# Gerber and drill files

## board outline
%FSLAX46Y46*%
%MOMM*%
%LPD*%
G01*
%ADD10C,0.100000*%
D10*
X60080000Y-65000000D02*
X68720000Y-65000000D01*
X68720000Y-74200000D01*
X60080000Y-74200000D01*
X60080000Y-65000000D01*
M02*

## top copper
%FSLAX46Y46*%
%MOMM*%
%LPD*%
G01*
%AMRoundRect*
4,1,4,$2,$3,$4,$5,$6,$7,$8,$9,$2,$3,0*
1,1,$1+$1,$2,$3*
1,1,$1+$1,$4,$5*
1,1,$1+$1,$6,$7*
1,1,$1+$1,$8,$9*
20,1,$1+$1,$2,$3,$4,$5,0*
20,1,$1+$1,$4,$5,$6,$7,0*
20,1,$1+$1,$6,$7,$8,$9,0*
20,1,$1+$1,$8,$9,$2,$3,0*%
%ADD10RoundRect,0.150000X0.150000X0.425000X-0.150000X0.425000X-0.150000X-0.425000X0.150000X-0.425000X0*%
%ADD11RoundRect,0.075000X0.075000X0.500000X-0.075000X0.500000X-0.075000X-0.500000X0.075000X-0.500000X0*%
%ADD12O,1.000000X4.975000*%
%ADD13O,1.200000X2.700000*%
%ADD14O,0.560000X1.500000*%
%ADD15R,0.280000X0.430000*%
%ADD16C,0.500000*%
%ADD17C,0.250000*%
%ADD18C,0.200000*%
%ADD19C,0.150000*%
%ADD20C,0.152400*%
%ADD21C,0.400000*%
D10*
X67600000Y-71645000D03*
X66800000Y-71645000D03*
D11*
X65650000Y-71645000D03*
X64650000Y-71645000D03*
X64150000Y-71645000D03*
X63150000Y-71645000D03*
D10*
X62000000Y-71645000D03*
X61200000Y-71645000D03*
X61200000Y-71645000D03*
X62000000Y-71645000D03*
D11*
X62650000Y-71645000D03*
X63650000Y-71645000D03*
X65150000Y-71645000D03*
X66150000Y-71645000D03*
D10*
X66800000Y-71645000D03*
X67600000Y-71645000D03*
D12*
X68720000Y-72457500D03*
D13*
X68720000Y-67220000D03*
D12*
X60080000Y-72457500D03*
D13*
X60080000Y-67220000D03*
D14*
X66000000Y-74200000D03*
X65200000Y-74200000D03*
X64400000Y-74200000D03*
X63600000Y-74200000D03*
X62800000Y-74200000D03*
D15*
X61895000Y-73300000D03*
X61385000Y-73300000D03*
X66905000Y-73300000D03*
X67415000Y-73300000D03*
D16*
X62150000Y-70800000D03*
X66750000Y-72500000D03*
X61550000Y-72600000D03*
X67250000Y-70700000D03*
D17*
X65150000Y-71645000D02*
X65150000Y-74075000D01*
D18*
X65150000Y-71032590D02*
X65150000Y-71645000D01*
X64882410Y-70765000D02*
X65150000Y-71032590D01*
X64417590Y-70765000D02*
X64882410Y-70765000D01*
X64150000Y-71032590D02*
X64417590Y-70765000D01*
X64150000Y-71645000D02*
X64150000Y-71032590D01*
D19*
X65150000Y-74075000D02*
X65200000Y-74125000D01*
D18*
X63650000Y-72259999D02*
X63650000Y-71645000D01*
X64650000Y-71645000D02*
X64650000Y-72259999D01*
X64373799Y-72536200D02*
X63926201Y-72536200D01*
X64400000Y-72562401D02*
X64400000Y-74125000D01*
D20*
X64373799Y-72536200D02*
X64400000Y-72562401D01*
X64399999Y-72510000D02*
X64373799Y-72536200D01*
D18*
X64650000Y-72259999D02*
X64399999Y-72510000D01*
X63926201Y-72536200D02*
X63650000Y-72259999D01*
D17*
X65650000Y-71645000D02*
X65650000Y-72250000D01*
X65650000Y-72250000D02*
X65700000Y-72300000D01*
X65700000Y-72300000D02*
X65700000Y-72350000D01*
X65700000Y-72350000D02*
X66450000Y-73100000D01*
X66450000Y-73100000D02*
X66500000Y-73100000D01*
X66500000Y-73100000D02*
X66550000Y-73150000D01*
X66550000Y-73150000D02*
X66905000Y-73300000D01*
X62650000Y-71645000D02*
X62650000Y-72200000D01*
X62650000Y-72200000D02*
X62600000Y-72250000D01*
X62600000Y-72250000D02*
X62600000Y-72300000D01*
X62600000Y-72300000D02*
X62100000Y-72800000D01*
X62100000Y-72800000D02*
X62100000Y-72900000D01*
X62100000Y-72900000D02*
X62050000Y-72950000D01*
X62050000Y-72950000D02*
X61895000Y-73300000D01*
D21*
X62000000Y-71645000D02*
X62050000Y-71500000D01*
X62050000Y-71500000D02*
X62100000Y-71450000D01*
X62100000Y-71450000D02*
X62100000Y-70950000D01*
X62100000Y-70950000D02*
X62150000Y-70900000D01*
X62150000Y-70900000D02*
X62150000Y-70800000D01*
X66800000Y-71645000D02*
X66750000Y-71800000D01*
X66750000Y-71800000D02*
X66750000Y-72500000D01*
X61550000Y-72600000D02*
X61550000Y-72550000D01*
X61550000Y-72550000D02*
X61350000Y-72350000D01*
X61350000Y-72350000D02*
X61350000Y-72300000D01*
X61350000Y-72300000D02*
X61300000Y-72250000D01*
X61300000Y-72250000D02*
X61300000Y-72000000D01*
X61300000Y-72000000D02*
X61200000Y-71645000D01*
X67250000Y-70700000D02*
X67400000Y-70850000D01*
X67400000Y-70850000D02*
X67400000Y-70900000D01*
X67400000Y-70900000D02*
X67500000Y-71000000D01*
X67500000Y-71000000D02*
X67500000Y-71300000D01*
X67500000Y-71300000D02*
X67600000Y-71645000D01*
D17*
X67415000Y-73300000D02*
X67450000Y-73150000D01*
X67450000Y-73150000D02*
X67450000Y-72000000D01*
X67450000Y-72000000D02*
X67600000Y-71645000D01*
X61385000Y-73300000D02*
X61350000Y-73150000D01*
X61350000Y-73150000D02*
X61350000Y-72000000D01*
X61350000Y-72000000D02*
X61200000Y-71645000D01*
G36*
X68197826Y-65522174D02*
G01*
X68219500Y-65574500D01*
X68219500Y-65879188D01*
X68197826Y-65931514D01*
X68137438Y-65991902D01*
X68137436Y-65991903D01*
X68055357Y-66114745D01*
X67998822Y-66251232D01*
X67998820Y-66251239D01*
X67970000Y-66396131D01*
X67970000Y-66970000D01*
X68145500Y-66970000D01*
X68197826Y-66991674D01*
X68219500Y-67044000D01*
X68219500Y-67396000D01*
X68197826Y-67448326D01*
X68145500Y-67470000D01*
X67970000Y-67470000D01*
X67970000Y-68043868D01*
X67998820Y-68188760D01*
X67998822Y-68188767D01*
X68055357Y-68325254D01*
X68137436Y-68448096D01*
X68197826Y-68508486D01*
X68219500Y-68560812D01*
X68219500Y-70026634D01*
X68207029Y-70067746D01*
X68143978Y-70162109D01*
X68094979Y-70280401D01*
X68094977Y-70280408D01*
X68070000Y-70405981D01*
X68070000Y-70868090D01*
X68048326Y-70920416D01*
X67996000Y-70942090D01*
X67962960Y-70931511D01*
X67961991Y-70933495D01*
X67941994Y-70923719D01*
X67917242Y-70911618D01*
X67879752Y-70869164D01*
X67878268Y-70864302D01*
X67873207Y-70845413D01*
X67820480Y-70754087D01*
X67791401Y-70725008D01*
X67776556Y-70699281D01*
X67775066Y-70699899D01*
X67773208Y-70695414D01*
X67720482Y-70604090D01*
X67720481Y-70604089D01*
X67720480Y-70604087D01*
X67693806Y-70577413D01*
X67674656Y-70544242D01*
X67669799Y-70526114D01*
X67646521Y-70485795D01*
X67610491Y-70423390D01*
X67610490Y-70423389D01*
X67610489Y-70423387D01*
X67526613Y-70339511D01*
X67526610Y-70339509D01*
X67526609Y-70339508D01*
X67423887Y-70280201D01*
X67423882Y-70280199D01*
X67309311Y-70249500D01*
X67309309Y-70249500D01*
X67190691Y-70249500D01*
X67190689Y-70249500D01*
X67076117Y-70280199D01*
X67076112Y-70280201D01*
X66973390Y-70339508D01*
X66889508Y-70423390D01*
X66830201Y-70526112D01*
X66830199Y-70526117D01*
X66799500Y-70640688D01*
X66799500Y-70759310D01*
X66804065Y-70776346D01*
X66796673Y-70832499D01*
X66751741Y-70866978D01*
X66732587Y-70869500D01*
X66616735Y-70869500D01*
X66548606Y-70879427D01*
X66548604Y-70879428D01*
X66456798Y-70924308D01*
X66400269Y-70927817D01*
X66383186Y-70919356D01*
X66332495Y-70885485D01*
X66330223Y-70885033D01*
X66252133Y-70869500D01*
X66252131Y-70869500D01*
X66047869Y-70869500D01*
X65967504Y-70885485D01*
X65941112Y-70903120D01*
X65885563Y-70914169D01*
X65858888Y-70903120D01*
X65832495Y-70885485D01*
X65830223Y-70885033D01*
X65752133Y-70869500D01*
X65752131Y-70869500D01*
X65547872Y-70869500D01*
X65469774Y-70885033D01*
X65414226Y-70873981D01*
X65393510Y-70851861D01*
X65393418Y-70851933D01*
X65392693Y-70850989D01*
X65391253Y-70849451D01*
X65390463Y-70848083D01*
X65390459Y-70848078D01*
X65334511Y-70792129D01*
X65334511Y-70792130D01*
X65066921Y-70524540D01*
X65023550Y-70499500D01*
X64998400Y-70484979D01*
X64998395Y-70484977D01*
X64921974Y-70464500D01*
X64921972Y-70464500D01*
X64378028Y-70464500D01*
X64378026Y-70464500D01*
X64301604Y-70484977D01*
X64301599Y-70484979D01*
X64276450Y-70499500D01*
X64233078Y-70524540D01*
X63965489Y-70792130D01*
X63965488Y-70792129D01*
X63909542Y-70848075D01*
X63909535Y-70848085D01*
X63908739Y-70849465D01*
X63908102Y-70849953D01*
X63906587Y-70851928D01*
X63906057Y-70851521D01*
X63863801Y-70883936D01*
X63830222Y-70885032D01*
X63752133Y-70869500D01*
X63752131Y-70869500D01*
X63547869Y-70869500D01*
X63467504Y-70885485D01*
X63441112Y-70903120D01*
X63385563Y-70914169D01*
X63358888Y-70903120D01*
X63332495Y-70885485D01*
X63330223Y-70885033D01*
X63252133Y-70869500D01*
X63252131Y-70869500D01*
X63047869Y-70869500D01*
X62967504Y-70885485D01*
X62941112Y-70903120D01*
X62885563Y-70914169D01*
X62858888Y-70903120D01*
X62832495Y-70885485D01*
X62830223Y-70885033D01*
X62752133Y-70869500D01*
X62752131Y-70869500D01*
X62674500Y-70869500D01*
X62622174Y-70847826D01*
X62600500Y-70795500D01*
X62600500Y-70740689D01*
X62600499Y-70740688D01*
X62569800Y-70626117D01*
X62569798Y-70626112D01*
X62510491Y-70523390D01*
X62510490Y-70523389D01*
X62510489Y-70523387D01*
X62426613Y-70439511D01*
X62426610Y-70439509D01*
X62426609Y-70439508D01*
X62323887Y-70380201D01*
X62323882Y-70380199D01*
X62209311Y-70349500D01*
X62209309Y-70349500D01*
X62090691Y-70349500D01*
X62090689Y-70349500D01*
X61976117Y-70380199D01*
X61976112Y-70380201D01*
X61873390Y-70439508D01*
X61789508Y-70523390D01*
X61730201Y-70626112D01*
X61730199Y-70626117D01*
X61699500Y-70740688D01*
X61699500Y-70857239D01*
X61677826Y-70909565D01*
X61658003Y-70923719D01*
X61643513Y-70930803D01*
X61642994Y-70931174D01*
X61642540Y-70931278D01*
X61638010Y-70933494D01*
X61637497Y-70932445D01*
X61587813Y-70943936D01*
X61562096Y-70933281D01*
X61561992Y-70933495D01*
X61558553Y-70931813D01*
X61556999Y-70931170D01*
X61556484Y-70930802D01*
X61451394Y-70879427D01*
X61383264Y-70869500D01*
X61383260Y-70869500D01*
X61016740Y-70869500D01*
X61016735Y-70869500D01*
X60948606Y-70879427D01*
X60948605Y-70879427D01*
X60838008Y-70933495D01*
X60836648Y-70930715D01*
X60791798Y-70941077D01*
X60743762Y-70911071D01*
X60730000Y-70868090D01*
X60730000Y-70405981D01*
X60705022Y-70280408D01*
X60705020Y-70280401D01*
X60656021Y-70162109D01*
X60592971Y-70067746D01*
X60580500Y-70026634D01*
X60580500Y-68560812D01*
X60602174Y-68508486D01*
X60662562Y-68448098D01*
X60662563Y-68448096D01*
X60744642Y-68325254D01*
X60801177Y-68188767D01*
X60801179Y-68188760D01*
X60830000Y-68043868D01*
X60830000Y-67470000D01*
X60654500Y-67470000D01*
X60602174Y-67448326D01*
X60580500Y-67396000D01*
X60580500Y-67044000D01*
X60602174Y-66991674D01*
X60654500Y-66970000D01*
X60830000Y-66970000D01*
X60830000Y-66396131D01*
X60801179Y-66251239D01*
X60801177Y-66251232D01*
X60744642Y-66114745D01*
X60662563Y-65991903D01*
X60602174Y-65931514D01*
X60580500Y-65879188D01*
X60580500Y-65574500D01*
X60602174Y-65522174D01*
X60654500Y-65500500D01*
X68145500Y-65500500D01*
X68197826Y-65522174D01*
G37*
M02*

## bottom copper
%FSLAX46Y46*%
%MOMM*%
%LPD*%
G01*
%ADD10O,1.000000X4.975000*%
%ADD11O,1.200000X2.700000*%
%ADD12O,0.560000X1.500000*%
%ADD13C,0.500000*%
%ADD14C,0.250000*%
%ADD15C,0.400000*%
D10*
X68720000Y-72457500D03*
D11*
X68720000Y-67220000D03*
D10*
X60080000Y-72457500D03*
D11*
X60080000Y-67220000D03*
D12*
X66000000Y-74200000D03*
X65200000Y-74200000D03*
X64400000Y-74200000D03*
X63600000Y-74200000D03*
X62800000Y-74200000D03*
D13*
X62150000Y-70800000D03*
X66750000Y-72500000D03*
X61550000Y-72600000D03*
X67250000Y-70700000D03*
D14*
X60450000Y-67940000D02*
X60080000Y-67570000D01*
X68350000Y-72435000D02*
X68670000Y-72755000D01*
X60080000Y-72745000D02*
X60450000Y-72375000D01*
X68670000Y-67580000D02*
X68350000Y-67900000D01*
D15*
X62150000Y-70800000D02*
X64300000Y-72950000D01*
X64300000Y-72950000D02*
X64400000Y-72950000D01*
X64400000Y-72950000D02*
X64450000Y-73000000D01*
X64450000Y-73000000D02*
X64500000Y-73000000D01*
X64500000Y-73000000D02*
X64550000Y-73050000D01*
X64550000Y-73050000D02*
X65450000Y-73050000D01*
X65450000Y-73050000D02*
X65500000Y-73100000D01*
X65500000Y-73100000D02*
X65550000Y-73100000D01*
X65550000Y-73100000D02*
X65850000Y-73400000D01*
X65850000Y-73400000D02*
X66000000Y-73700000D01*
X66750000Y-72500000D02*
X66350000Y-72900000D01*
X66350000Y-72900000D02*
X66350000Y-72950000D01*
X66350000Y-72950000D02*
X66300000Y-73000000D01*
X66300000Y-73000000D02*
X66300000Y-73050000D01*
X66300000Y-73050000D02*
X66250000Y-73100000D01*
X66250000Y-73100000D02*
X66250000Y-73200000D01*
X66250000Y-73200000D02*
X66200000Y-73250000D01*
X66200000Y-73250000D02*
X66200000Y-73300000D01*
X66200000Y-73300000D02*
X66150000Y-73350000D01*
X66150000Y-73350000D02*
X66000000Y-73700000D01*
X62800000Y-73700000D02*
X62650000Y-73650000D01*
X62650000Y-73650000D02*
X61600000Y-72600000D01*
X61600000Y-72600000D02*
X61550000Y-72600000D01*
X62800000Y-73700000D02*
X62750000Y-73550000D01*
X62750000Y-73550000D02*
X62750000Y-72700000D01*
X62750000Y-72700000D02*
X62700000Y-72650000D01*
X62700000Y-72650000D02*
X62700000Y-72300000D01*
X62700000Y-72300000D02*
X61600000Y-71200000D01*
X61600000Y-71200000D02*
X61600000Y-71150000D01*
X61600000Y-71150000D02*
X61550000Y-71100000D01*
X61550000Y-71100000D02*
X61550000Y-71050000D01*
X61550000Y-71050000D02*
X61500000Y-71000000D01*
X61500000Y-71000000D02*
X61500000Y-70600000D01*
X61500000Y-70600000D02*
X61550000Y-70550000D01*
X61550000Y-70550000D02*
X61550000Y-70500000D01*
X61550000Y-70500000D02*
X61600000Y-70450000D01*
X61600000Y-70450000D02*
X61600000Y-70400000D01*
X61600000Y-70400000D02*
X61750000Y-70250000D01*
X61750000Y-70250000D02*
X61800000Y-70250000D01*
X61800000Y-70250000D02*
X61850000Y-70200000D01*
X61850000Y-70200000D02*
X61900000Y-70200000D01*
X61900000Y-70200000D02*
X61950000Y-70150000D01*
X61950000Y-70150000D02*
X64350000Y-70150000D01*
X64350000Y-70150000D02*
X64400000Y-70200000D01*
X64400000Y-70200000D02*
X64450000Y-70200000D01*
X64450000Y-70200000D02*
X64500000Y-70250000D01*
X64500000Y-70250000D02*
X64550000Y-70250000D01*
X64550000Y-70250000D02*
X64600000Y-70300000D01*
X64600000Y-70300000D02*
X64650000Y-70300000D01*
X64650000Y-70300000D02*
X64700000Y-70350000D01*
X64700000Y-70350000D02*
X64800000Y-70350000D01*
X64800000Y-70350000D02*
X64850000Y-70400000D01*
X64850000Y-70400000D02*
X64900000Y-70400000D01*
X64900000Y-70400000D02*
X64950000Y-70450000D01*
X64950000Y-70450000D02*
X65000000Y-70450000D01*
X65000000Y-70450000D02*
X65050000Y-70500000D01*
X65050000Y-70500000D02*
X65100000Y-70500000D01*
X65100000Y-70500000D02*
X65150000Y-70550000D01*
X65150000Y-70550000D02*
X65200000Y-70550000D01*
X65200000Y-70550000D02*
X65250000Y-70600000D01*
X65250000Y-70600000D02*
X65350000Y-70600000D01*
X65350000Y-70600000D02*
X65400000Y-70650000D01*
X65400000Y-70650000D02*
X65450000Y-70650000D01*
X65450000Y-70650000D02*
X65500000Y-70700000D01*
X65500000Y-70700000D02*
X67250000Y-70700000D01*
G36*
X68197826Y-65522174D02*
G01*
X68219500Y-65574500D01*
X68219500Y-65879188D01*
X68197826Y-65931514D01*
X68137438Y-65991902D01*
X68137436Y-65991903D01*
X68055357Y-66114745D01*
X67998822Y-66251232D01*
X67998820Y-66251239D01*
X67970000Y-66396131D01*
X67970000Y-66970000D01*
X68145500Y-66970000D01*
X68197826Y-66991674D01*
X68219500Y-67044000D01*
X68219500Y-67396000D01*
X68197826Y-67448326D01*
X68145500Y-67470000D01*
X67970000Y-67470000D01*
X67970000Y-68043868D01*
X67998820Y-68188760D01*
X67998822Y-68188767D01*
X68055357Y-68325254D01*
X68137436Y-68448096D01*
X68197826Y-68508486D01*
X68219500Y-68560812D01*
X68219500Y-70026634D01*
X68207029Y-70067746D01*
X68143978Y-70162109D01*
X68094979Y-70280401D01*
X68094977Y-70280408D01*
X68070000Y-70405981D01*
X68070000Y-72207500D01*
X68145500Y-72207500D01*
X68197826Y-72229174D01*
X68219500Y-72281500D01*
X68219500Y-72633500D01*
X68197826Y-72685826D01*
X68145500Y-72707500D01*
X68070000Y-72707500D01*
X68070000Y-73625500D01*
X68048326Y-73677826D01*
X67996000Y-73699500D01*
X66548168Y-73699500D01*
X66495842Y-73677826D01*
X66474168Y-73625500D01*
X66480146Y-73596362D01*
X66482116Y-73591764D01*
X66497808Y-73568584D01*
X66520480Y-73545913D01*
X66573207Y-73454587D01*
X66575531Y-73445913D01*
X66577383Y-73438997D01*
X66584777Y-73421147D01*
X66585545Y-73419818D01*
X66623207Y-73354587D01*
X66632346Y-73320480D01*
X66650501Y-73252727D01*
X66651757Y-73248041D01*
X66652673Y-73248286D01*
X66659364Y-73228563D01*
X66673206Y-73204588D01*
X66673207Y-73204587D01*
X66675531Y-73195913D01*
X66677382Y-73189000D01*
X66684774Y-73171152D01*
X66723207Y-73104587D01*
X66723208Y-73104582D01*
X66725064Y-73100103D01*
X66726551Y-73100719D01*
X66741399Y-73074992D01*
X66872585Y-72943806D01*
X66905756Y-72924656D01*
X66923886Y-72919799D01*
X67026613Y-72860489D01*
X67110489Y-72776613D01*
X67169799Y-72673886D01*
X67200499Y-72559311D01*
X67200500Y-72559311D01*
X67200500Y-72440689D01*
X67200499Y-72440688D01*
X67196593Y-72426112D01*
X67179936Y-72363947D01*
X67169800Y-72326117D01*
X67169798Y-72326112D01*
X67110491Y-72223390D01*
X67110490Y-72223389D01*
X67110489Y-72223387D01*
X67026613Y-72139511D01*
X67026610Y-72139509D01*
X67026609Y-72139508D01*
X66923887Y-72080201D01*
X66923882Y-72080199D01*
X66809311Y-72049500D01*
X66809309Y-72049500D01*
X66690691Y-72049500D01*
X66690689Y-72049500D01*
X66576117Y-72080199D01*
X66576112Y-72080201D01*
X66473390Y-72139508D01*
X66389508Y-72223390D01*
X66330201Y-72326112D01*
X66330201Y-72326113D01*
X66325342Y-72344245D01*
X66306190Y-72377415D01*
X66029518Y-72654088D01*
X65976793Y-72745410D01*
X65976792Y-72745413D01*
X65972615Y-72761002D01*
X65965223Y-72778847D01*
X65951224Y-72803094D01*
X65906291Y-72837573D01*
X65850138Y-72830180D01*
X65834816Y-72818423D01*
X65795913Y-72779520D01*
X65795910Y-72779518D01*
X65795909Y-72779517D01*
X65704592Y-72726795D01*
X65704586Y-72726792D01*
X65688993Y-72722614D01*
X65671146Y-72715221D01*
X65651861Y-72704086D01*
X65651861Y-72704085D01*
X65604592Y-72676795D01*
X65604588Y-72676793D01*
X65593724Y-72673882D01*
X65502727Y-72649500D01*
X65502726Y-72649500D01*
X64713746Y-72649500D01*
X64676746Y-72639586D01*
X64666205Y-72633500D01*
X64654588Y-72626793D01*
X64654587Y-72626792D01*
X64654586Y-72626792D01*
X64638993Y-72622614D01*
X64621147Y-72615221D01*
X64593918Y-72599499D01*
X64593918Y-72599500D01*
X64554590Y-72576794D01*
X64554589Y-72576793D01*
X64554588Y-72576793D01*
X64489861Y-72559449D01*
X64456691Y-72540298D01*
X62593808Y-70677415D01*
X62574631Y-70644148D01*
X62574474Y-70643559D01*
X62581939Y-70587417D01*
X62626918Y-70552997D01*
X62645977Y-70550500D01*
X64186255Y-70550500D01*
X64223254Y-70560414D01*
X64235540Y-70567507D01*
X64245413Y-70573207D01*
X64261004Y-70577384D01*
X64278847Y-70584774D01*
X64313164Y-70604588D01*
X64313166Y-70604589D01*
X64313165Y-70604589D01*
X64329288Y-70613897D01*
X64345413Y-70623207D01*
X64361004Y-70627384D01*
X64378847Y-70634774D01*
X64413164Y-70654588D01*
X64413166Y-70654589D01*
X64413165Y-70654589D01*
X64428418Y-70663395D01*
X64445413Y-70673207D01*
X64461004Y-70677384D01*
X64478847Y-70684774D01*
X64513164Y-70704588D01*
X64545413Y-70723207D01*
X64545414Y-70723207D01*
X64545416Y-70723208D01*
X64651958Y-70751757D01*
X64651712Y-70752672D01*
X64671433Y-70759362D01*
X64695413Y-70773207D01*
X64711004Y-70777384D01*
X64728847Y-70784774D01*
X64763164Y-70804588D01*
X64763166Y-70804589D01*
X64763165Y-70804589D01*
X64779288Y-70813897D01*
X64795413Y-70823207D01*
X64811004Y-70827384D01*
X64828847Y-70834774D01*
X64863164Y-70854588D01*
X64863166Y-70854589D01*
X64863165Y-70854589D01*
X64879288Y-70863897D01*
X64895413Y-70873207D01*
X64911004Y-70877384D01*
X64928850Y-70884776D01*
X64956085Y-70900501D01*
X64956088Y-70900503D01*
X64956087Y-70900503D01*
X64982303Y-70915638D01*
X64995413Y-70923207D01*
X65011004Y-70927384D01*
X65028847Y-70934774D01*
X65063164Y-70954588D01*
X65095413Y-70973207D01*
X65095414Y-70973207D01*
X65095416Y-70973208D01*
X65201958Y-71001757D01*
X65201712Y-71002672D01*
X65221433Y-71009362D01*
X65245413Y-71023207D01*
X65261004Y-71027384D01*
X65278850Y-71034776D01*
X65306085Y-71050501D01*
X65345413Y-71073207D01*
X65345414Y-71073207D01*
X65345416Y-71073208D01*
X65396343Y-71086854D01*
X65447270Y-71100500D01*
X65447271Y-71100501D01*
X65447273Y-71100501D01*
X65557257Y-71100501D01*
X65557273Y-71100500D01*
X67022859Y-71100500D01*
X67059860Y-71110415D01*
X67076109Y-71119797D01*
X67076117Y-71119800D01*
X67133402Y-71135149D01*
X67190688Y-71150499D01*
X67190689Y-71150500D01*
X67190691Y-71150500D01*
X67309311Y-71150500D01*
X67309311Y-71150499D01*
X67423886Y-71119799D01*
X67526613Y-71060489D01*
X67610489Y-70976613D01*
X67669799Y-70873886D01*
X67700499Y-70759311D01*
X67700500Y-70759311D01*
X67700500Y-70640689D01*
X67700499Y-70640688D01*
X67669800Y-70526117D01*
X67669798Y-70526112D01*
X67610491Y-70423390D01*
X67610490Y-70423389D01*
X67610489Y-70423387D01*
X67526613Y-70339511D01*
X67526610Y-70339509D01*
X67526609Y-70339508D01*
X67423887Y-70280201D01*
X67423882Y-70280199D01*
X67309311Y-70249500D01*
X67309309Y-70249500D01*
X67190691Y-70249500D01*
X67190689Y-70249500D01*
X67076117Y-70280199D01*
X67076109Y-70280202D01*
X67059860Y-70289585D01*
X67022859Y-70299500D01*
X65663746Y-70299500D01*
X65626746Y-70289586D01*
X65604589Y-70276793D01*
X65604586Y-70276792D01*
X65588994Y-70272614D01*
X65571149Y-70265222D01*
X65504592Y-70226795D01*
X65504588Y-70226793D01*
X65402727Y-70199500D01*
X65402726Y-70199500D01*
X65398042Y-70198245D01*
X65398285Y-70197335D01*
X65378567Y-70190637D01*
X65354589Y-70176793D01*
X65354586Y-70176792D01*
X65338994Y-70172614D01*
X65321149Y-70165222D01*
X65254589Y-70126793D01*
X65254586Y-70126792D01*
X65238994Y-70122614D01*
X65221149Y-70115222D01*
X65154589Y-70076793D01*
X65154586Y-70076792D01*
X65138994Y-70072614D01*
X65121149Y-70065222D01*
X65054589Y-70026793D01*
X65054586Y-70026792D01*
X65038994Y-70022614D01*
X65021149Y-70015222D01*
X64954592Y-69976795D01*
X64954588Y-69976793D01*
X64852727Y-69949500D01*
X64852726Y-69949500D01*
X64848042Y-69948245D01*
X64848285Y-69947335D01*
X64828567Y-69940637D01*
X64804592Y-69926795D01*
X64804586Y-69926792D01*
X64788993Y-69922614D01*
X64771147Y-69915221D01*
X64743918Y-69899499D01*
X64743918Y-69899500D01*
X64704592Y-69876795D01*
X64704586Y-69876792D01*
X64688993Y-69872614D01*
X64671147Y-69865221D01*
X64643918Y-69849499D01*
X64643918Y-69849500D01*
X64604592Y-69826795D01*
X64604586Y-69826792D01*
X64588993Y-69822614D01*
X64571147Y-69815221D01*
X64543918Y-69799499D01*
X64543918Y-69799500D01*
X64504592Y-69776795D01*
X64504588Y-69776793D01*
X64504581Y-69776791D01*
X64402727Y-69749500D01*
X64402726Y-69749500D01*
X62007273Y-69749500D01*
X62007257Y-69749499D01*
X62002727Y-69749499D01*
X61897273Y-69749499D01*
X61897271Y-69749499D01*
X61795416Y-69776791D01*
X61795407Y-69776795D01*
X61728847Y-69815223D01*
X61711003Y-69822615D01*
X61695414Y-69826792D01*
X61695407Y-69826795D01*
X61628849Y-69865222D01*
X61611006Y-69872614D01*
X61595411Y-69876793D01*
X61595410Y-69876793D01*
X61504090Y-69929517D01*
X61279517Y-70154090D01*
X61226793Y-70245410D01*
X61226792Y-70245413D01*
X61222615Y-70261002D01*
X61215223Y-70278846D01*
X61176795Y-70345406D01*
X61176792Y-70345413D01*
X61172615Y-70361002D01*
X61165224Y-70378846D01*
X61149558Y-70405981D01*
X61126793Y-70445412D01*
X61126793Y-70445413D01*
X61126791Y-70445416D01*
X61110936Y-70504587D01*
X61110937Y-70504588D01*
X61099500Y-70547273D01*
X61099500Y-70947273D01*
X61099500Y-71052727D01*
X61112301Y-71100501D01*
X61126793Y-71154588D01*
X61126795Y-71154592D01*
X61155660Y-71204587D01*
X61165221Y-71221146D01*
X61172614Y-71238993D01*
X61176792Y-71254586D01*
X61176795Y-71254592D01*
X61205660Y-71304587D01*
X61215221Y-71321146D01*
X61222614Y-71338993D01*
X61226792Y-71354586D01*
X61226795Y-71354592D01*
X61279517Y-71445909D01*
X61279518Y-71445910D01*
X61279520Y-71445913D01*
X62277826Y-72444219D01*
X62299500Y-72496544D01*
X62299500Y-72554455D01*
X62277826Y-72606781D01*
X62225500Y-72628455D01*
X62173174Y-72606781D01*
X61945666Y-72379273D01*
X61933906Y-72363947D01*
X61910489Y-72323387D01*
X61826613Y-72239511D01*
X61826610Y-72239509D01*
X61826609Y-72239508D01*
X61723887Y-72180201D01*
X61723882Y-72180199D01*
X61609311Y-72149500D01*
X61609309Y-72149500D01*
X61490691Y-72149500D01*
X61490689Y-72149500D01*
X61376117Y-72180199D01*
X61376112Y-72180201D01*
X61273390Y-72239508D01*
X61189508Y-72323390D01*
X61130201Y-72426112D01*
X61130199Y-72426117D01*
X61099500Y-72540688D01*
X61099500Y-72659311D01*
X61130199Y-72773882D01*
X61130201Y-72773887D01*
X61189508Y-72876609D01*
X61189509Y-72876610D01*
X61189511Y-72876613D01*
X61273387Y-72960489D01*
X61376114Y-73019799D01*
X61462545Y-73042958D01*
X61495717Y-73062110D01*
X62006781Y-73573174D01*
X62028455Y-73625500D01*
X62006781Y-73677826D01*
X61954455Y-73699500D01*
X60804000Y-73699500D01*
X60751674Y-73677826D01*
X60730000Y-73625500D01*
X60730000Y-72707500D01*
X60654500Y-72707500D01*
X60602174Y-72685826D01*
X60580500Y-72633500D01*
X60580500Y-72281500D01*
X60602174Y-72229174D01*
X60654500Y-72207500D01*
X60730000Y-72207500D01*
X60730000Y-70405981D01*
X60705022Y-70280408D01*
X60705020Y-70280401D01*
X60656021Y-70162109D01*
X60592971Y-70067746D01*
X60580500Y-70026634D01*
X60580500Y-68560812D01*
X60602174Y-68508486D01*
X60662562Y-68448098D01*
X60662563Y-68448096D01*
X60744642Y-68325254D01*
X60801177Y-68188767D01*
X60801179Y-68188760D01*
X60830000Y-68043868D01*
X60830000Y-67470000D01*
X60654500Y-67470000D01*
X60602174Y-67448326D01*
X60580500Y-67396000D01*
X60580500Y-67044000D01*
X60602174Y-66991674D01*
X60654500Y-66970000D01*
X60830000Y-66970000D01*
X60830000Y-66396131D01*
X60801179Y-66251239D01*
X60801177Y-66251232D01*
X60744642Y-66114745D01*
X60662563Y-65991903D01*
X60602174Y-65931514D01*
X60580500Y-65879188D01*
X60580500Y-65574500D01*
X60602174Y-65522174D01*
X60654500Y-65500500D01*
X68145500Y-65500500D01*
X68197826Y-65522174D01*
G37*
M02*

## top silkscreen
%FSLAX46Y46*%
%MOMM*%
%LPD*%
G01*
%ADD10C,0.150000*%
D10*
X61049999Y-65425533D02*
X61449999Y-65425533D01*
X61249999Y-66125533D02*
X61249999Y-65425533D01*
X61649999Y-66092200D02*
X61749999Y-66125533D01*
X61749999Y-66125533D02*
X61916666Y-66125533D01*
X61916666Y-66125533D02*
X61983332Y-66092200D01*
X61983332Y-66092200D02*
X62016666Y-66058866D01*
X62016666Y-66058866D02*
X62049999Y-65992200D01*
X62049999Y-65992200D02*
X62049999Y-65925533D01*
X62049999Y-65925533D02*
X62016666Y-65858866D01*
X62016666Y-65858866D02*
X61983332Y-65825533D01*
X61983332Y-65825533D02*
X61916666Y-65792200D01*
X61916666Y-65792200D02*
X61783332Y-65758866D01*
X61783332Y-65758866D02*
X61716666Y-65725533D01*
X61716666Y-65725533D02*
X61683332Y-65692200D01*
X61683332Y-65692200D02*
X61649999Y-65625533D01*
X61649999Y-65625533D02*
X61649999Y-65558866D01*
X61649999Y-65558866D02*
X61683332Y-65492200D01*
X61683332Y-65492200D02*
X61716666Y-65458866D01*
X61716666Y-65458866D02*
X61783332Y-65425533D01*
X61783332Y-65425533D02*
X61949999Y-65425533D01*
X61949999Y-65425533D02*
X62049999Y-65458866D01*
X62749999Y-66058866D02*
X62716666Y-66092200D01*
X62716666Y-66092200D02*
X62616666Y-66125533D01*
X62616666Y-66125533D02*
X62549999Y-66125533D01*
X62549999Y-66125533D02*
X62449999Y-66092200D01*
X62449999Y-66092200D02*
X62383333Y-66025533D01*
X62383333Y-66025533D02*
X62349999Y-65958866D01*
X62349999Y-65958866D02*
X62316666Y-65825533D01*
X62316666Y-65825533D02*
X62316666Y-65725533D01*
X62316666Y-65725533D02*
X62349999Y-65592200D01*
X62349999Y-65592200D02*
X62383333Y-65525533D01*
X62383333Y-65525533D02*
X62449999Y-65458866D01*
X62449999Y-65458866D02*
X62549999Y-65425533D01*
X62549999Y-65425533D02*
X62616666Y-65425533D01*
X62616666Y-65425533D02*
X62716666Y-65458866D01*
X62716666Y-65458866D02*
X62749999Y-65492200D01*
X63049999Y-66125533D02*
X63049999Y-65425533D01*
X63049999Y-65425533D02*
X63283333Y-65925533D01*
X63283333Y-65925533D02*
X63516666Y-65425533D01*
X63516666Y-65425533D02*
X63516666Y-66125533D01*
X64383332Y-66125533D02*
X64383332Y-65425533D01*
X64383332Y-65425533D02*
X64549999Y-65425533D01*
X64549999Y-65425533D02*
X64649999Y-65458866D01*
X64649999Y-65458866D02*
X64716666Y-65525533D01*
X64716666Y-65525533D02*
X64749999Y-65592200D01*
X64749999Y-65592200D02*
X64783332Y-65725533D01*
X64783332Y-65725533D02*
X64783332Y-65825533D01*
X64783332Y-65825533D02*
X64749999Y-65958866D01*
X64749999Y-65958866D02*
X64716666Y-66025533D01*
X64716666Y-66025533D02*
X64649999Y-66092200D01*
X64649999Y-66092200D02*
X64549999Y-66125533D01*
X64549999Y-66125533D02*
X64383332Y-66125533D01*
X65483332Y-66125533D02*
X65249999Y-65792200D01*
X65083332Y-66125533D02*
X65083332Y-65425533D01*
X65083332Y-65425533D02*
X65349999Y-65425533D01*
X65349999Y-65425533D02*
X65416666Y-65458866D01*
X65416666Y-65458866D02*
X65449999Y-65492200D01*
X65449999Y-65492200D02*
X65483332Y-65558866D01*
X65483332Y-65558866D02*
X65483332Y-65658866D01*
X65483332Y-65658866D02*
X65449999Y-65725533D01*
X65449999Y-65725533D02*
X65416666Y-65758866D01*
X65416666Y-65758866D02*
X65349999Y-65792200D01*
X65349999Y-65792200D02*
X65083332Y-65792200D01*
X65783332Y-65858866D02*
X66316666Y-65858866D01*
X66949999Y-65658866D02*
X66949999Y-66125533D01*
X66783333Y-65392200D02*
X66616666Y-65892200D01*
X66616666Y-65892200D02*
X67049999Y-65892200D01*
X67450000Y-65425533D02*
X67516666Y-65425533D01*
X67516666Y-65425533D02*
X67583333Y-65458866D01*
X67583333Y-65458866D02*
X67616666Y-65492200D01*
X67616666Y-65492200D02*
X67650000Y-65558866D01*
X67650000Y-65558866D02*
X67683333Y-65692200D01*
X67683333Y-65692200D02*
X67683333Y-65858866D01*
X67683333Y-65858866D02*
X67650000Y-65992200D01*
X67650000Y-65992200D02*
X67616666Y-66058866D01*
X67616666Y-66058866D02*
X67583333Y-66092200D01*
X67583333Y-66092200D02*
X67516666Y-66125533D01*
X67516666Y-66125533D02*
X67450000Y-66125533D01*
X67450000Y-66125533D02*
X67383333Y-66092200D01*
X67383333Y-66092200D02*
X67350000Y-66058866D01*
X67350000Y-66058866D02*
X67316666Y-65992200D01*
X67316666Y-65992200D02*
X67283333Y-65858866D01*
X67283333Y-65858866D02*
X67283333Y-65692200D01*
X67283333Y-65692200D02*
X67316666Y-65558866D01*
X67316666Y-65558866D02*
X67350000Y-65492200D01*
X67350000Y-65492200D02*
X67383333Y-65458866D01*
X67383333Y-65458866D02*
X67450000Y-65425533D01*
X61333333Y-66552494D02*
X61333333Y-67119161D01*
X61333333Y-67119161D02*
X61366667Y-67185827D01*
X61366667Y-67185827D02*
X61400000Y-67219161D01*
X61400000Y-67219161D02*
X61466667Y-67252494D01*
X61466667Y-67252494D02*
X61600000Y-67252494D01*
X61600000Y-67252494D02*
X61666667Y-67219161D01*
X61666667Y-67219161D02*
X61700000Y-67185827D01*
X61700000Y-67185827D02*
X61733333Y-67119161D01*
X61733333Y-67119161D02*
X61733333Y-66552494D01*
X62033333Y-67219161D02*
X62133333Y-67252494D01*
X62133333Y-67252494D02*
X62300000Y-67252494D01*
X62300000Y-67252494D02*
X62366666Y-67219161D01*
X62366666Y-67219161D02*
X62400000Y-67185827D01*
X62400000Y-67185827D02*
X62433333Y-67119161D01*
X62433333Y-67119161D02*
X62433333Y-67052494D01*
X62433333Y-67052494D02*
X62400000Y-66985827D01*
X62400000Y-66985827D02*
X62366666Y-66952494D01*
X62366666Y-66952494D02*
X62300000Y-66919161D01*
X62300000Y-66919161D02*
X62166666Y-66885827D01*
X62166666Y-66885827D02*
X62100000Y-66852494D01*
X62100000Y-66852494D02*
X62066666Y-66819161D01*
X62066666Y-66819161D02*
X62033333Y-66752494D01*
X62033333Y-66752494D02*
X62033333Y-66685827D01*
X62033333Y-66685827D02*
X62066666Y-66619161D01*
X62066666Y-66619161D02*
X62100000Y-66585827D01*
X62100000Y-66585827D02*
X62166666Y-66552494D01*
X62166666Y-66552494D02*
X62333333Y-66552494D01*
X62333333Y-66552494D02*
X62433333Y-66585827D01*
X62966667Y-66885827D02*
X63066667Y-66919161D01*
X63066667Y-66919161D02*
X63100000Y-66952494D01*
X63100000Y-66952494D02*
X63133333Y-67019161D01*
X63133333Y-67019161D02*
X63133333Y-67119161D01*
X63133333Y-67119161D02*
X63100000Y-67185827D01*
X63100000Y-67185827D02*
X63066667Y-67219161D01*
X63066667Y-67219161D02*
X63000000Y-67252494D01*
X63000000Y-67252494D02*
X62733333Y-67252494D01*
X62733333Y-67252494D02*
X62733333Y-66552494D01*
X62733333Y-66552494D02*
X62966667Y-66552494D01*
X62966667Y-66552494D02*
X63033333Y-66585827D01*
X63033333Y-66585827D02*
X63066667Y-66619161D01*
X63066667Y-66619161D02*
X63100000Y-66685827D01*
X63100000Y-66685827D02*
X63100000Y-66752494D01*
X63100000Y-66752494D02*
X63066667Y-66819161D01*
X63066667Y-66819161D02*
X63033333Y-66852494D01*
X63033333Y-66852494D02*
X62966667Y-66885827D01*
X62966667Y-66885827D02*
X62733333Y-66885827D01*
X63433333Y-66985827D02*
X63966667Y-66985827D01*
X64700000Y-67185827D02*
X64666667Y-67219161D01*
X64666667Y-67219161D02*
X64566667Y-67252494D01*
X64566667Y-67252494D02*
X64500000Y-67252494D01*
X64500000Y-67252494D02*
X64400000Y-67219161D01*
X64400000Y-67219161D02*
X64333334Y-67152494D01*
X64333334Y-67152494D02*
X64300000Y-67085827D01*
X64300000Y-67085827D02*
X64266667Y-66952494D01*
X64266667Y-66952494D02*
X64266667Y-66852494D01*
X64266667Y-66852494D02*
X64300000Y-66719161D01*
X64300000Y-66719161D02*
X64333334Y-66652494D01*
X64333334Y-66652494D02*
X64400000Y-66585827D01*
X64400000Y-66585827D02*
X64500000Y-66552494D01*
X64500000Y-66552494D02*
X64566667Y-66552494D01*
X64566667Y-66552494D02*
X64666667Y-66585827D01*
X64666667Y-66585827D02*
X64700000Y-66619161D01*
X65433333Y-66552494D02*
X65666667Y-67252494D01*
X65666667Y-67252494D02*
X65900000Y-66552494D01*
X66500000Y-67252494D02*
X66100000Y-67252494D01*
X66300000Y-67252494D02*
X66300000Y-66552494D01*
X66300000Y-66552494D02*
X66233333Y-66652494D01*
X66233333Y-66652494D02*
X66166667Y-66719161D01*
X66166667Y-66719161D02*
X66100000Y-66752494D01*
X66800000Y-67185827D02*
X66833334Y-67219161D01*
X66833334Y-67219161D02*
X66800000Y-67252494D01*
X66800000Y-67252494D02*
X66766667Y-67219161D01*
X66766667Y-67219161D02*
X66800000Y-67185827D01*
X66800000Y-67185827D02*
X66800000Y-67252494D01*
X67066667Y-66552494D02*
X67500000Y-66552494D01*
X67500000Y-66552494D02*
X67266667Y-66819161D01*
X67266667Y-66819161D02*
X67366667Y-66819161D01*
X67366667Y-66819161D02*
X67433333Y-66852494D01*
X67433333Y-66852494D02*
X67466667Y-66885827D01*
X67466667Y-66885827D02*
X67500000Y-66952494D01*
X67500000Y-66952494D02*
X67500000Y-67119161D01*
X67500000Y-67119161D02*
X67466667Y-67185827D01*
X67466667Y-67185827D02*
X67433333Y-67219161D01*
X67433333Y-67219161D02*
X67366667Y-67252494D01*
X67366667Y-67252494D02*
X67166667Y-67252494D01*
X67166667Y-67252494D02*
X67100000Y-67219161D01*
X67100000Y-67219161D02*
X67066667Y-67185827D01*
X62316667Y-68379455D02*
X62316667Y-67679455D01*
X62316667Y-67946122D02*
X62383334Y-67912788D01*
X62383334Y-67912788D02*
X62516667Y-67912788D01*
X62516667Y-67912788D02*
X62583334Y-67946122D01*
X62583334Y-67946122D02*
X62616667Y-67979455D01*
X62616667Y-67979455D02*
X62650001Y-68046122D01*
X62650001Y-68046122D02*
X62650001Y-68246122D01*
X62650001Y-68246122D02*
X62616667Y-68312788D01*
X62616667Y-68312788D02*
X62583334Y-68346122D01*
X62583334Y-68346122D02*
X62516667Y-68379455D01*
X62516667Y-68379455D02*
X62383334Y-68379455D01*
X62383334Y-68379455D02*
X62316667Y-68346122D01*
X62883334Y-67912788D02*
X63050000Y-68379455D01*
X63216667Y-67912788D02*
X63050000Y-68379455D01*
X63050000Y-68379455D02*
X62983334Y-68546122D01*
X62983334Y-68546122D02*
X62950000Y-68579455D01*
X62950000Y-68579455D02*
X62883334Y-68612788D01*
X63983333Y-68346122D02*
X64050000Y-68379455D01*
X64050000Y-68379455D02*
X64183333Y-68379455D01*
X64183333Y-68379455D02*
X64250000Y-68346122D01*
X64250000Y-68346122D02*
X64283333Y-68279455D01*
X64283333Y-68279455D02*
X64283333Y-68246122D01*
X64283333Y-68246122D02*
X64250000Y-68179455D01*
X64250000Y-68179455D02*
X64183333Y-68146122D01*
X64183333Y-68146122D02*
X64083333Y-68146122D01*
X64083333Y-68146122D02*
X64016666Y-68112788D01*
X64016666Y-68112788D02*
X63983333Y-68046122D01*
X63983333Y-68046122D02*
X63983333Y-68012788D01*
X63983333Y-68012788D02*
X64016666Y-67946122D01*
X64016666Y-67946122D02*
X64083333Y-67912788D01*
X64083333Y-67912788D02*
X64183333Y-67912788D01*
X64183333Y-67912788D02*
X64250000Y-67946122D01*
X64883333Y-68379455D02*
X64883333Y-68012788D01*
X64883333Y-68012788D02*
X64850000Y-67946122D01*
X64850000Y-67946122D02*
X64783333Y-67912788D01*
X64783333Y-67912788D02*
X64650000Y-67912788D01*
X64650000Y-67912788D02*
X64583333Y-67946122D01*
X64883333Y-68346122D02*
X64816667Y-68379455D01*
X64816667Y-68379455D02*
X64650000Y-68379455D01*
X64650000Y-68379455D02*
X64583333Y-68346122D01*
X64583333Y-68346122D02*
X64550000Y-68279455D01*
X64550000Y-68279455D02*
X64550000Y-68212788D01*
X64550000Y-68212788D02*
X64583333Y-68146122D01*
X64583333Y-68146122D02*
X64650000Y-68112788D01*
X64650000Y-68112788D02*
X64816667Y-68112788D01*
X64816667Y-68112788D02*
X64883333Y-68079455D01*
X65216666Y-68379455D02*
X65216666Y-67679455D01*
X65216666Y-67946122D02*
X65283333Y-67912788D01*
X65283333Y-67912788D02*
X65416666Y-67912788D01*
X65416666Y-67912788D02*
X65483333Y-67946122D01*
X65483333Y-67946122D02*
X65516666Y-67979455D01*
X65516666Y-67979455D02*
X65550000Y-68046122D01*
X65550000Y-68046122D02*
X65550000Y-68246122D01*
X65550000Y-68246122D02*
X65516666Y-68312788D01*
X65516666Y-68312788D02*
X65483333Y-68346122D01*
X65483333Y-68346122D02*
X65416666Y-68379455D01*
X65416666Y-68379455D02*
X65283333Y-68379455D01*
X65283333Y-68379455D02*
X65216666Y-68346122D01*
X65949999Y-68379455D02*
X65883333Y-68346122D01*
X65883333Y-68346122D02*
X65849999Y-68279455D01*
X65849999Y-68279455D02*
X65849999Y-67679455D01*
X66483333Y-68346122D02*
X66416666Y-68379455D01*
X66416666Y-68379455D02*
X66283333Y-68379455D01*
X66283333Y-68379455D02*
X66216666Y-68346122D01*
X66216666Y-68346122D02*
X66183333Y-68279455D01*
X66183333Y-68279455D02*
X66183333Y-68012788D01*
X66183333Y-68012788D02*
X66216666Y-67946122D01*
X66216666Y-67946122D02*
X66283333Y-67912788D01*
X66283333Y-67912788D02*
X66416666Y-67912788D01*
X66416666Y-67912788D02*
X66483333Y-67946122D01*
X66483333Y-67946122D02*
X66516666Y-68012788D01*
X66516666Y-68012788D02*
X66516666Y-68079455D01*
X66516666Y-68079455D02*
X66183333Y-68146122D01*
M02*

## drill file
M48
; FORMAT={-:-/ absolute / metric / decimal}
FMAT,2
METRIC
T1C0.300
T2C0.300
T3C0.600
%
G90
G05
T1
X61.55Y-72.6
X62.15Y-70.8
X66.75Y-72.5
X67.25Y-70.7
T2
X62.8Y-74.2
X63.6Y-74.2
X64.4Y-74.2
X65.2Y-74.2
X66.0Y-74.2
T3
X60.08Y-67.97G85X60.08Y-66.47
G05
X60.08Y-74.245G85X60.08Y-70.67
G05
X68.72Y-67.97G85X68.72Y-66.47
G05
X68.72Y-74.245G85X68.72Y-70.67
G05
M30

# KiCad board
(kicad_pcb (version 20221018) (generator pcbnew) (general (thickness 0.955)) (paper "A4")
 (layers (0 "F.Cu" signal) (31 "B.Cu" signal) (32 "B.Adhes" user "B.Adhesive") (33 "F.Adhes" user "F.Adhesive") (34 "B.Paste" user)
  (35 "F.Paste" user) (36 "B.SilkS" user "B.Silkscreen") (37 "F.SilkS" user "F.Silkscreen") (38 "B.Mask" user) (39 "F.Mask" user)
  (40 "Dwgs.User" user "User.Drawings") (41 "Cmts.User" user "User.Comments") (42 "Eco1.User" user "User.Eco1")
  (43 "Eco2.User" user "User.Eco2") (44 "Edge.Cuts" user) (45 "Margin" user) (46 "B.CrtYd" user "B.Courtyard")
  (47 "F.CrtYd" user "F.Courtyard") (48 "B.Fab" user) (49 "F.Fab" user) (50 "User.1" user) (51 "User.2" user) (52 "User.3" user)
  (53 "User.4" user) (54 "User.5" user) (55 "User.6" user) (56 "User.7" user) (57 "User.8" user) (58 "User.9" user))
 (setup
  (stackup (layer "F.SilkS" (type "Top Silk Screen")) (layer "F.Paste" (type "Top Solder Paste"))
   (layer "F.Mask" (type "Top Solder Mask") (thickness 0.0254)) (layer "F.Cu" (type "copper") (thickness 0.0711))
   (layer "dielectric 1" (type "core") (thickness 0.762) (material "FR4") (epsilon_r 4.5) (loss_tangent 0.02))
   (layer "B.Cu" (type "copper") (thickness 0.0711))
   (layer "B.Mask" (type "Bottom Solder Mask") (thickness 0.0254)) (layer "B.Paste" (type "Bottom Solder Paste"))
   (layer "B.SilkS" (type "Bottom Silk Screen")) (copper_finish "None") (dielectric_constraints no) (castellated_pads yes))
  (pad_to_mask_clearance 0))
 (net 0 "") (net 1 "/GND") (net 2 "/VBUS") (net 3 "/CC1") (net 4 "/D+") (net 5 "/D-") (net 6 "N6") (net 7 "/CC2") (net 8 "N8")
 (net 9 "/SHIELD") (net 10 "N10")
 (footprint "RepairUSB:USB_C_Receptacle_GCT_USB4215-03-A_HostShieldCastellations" (layer "F.Cu") (at 64.4 68.645 180)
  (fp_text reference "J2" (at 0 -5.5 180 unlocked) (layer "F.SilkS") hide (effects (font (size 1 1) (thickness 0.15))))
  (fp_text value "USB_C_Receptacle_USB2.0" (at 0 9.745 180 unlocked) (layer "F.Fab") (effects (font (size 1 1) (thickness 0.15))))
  (pad "A1" smd roundrect (at -3.2 -3 180) (size 0.6 1.15) (layers "F.Cu" "F.Paste" "F.Mask") (roundrect_rratio 0.25) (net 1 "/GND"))
  (pad "A4" smd roundrect (at -2.4 -3 180) (size 0.6 1.15) (layers "F.Cu" "F.Paste" "F.Mask") (roundrect_rratio 0.25) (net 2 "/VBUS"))
  (pad "A5" smd roundrect (at -1.25 -3 180) (size 0.3 1.15) (layers "F.Cu" "F.Paste" "F.Mask") (roundrect_rratio 0.25) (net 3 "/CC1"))
  (pad "A6" smd roundrect (at -0.25 -3 180) (size 0.3 1.15) (layers "F.Cu" "F.Paste" "F.Mask") (roundrect_rratio 0.25) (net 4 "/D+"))
  (pad "A7" smd roundrect (at 0.25 -3 180) (size 0.3 1.15) (layers "F.Cu" "F.Paste" "F.Mask") (roundrect_rratio 0.25) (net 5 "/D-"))
  (pad "A8" smd roundrect (at 1.25 -3 180) (size 0.3 1.15) (layers "F.Cu" "F.Paste" "F.Mask") (roundrect_rratio 0.25) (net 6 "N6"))
  (pad "A9" smd roundrect (at 2.4 -3 180) (size 0.6 1.15) (layers "F.Cu" "F.Paste" "F.Mask") (roundrect_rratio 0.25) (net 2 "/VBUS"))
  (pad "A12" smd roundrect (at 3.2 -3 180) (size 0.6 1.15) (layers "F.Cu" "F.Paste" "F.Mask") (roundrect_rratio 0.25) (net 1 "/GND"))
  (pad "B1" smd roundrect (at 3.2 -3 180) (size 0.6 1.15) (layers "F.Cu" "F.Paste" "F.Mask") (roundrect_rratio 0.25) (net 1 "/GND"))
  (pad "B4" smd roundrect (at 2.4 -3 180) (size 0.6 1.15) (layers "F.Cu" "F.Paste" "F.Mask") (roundrect_rratio 0.25) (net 2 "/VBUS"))
  (pad "B5" smd roundrect (at 1.75 -3 180) (size 0.3 1.15) (layers "F.Cu" "F.Paste" "F.Mask") (roundrect_rratio 0.25) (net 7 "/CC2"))
  (pad "B6" smd roundrect (at 0.75 -3 180) (size 0.3 1.15) (layers "F.Cu" "F.Paste" "F.Mask") (roundrect_rratio 0.25) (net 4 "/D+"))
  (pad "B7" smd roundrect (at -0.75 -3 180) (size 0.3 1.15) (layers "F.Cu" "F.Paste" "F.Mask") (roundrect_rratio 0.25) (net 5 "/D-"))
  (pad "B8" smd roundrect (at -1.75 -3 180) (size 0.3 1.15) (layers "F.Cu" "F.Paste" "F.Mask") (roundrect_rratio 0.25) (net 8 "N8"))
  (pad "B9" smd roundrect (at -2.4 -3 180) (size 0.6 1.15) (layers "F.Cu" "F.Paste" "F.Mask") (roundrect_rratio 0.25) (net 2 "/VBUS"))
  (pad "B12" smd roundrect (at -3.2 -3 180) (size 0.6 1.15) (layers "F.Cu" "F.Paste" "F.Mask") (roundrect_rratio 0.25) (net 1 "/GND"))
  (pad "S1" thru_hole oval (at -4.32 -3.8125 180) (size 1 4.975) (drill oval 0.6 4.175) (layers "*.Cu" "*.Mask" "F.Paste") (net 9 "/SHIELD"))
  (pad "S1" thru_hole oval (at -4.32 1.425 180) (size 1.2 2.7) (drill oval 0.6 2.1) (layers "*.Cu" "*.Mask" "F.Paste") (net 9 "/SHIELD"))
  (pad "S1" thru_hole oval (at 4.32 -3.8125 180) (size 1 4.975) (drill oval 0.6 4.175) (layers "*.Cu" "*.Mask" "F.Paste") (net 9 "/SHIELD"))
  (pad "S1" thru_hole oval (at 4.32 1.425 180) (size 1.2 2.7) (drill oval 0.6 2.1) (layers "*.Cu" "*.Mask" "F.Paste") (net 9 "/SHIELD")))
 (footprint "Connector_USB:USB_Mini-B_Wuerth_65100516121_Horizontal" (layer "F.Cu") (at 64.4 72.35 180)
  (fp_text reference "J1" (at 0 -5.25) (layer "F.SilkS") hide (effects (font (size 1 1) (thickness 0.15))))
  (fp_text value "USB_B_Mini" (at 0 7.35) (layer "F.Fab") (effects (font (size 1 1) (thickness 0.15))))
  (pad "1" thru_hole oval (at -1.6 -1.85 180) (size 0.56 1.5) (drill 0.3) (layers "*.Cu" "*.Mask") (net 2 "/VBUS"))
  (pad "2" thru_hole oval (at -0.8 -1.85 180) (size 0.56 1.5) (drill 0.3) (layers "*.Cu" "*.Mask") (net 5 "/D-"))
  (pad "3" thru_hole oval (at 0 -1.85 180) (size 0.56 1.5) (drill 0.3) (layers "*.Cu" "*.Mask") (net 4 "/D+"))
  (pad "4" thru_hole oval (at 0.8 -1.85 180) (size 0.56 1.5) (drill 0.3) (layers "*.Cu" "*.Mask") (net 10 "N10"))
  (pad "5" thru_hole oval (at 1.6 -1.85 180) (size 0.56 1.5) (drill 0.3) (layers "*.Cu" "*.Mask") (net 1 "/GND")))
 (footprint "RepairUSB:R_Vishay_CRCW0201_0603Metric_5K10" (layer "F.Cu") (at 61.64 73.3 180)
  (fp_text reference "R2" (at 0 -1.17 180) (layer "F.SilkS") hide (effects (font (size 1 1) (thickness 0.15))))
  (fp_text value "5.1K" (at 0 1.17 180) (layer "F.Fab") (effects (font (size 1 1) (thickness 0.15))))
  (pad "1" smd rect (at -0.255 0 180) (size 0.28 0.43) (layers "F.Cu" "F.Paste" "F.Mask") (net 7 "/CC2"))
  (pad "2" smd rect (at 0.255 0 180) (size 0.28 0.43) (layers "F.Cu" "F.Paste" "F.Mask") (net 1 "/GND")))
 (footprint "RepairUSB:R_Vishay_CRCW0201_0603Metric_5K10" (layer "F.Cu") (at 67.16 73.3)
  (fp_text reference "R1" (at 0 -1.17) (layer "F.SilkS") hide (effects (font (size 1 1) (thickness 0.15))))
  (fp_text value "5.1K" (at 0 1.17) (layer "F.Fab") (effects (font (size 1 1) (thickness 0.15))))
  (pad "1" smd rect (at -0.255 0) (size 0.28 0.43) (layers "F.Cu" "F.Paste" "F.Mask") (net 3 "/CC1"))
  (pad "2" smd rect (at 0.255 0) (size 0.28 0.43) (layers "F.Cu" "F.Paste" "F.Mask") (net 1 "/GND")))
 (gr_rect locked (start 60.08 65) (end 68.72 74.2) (stroke (width 0.1) (type default)) (fill none) (layer "Edge.Cuts"))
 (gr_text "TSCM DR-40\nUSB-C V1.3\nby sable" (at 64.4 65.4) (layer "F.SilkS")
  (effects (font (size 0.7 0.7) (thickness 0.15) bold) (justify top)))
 (segment (start 65.15 71.645) (end 65.15 74.075) (width 0.25) (layer "F.Cu") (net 5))
 (segment (start 65.15 71.03259) (end 65.15 71.645) (width 0.2) (layer "F.Cu") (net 5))
 (segment (start 64.88241 70.765) (end 65.15 71.03259) (width 0.2) (layer "F.Cu") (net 5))
 (segment (start 64.41759 70.765) (end 64.88241 70.765) (width 0.2) (layer "F.Cu") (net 5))
 (segment (start 64.15 71.03259) (end 64.41759 70.765) (width 0.2) (layer "F.Cu") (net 5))
 (segment (start 64.15 71.645) (end 64.15 71.03259) (width 0.2) (layer "F.Cu") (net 5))
 (segment (start 65.15 74.075) (end 65.2 74.125) (width 0.15) (layer "F.Cu") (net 5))
 (segment (start 63.65 72.259999) (end 63.65 71.645) (width 0.2) (layer "F.Cu") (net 4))
 (segment (start 64.65 71.645) (end 64.65 72.259999) (width 0.2) (layer "F.Cu") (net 4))
 (segment (start 64.373799 72.5362) (end 63.926201 72.5362) (width 0.2) (layer "F.Cu") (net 4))
 (segment (start 64.4 72.562401) (end 64.4 74.125) (width 0.2) (layer "F.Cu") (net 4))
 (segment (start 64.373799 72.5362) (end 64.4 72.562401) (width 0.1524) (layer "F.Cu") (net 4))
 (segment (start 64.399999 72.51) (end 64.373799 72.5362) (width 0.1524) (layer "F.Cu") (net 4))
 (segment (start 64.65 72.259999) (end 64.399999 72.51) (width 0.2) (layer "F.Cu") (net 4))
 (segment (start 63.926201 72.5362) (end 63.65 72.259999) (width 0.2) (layer "F.Cu") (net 4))
 (segment (start 60.45 67.94) (end 60.08 67.57) (width 0.25) (layer "B.Cu") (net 9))
 (segment (start 68.35 72.435) (end 68.67 72.755) (width 0.25) (layer "B.Cu") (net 9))
 (segment (start 60.08 72.745) (end 60.45 72.375) (width 0.25) (layer "B.Cu") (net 9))
 (segment (start 68.67 67.58) (end 68.35 67.9) (width 0.25) (layer "B.Cu") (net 9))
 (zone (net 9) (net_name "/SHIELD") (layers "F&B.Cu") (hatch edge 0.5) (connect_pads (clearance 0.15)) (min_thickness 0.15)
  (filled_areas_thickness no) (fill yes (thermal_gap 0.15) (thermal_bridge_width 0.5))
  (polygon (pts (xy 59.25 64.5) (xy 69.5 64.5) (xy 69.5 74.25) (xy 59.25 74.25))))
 (segment (start 65.65 71.645) (end 65.65 72.25) (width 0.25) (layer "F.Cu") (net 3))
 (segment (start 65.65 72.25) (end 65.7 72.3) (width 0.25) (layer "F.Cu") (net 3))
 (segment (start 65.7 72.3) (end 65.7 72.35) (width 0.25) (layer "F.Cu") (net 3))
 (segment (start 65.7 72.35) (end 66.45 73.1) (width 0.25) (layer "F.Cu") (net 3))
 (segment (start 66.45 73.1) (end 66.5 73.1) (width 0.25) (layer "F.Cu") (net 3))
 (segment (start 66.5 73.1) (end 66.55 73.15) (width 0.25) (layer "F.Cu") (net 3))
 (segment (start 66.55 73.15) (end 66.905 73.3) (width 0.25) (layer "F.Cu") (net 3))
 (segment (start 62.65 71.645) (end 62.65 72.2) (width 0.25) (layer "F.Cu") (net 7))
 (segment (start 62.65 72.2) (end 62.6 72.25) (width 0.25) (layer "F.Cu") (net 7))
 (segment (start 62.6 72.25) (end 62.6 72.3) (width 0.25) (layer "F.Cu") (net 7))
 (segment (start 62.6 72.3) (end 62.1 72.8) (width 0.25) (layer "F.Cu") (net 7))
 (segment (start 62.1 72.8) (end 62.1 72.9) (width 0.25) (layer "F.Cu") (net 7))
 (segment (start 62.1 72.9) (end 62.05 72.95) (width 0.25) (layer "F.Cu") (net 7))
 (segment (start 62.05 72.95) (end 61.895 73.3) (width 0.25) (layer "F.Cu") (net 7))
 (segment (start 62 71.645) (end 62.05 71.5) (width 0.4) (layer "F.Cu") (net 2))
 (segment (start 62.05 71.5) (end 62.1 71.45) (width 0.4) (layer "F.Cu") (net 2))
 (segment (start 62.1 71.45) (end 62.1 70.95) (width 0.4) (layer "F.Cu") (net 2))
 (segment (start 62.1 70.95) (end 62.15 70.9) (width 0.4) (layer "F.Cu") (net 2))
 (segment (start 62.15 70.9) (end 62.15 70.8) (width 0.4) (layer "F.Cu") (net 2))
 (segment (start 62.15 70.8) (end 64.3 72.95) (width 0.4) (layer "B.Cu") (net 2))
 (segment (start 64.3 72.95) (end 64.4 72.95) (width 0.4) (layer "B.Cu") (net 2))
 (segment (start 64.4 72.95) (end 64.45 73) (width 0.4) (layer "B.Cu") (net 2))
 (segment (start 64.45 73) (end 64.5 73) (width 0.4) (layer "B.Cu") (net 2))
 (segment (start 64.5 73) (end 64.55 73.05) (width 0.4) (layer "B.Cu") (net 2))
 (segment (start 64.55 73.05) (end 65.45 73.05) (width 0.4) (layer "B.Cu") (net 2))
 (segment (start 65.45 73.05) (end 65.5 73.1) (width 0.4) (layer "B.Cu") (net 2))
 (segment (start 65.5 73.1) (end 65.55 73.1) (width 0.4) (layer "B.Cu") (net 2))
 (segment (start 65.55 73.1) (end 65.85 73.4) (width 0.4) (layer "B.Cu") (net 2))
 (segment (start 65.85 73.4) (end 66 73.7) (width 0.4) (layer "B.Cu") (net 2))
 (via (at 62.15 70.8) (size 0.5) (drill 0.3) (layers "F.Cu" "B.Cu") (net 2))
 (segment (start 66.8 71.645) (end 66.75 71.8) (width 0.4) (layer "F.Cu") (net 2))
 (segment (start 66.75 71.8) (end 66.75 72.5) (width 0.4) (layer "F.Cu") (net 2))
 (segment (start 66.75 72.5) (end 66.35 72.9) (width 0.4) (layer "B.Cu") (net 2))
 (segment (start 66.35 72.9) (end 66.35 72.95) (width 0.4) (layer "B.Cu") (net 2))
 (segment (start 66.35 72.95) (end 66.3 73) (width 0.4) (layer "B.Cu") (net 2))
 (segment (start 66.3 73) (end 66.3 73.05) (width 0.4) (layer "B.Cu") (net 2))
 (segment (start 66.3 73.05) (end 66.25 73.1) (width 0.4) (layer "B.Cu") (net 2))
 (segment (start 66.25 73.1) (end 66.25 73.2) (width 0.4) (layer "B.Cu") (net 2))
 (segment (start 66.25 73.2) (end 66.2 73.25) (width 0.4) (layer "B.Cu") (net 2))
 (segment (start 66.2 73.25) (end 66.2 73.3) (width 0.4) (layer "B.Cu") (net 2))
 (segment (start 66.2 73.3) (end 66.15 73.35) (width 0.4) (layer "B.Cu") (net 2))
 (segment (start 66.15 73.35) (end 66 73.7) (width 0.4) (layer "B.Cu") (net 2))
 (via (at 66.75 72.5) (size 0.5) (drill 0.3) (layers "F.Cu" "B.Cu") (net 2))
 (segment (start 62.8 73.7) (end 62.65 73.65) (width 0.4) (layer "B.Cu") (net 1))
 (segment (start 62.65 73.65) (end 61.6 72.6) (width 0.4) (layer "B.Cu") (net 1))
 (segment (start 61.6 72.6) (end 61.55 72.6) (width 0.4) (layer "B.Cu") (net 1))
 (segment (start 61.55 72.6) (end 61.55 72.55) (width 0.4) (layer "F.Cu") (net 1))
 (segment (start 61.55 72.55) (end 61.35 72.35) (width 0.4) (layer "F.Cu") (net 1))
 (segment (start 61.35 72.35) (end 61.35 72.3) (width 0.4) (layer "F.Cu") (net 1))
 (segment (start 61.35 72.3) (end 61.3 72.25) (width 0.4) (layer "F.Cu") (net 1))
 (segment (start 61.3 72.25) (end 61.3 72) (width 0.4) (layer "F.Cu") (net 1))
 (segment (start 61.3 72) (end 61.2 71.645) (width 0.4) (layer "F.Cu") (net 1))
 (via (at 61.55 72.6) (size 0.5) (drill 0.3) (layers "F.Cu" "B.Cu") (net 1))
 (segment (start 62.8 73.7) (end 62.75 73.55) (width 0.4) (layer "B.Cu") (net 1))
 (segment (start 62.75 73.55) (end 62.75 72.7) (width 0.4) (layer "B.Cu") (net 1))
 (segment (start 62.75 72.7) (end 62.7 72.65) (width 0.4) (layer "B.Cu") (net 1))
 (segment (start 62.7 72.65) (end 62.7 72.3) (width 0.4) (layer "B.Cu") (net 1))
 (segment (start 62.7 72.3) (end 61.6 71.2) (width 0.4) (layer "B.Cu") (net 1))
 (segment (start 61.6 71.2) (end 61.6 71.15) (width 0.4) (layer "B.Cu") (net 1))
 (segment (start 61.6 71.15) (end 61.55 71.1) (width 0.4) (layer "B.Cu") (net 1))
 (segment (start 61.55 71.1) (end 61.55 71.05) (width 0.4) (layer "B.Cu") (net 1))
 (segment (start 61.55 71.05) (end 61.5 71) (width 0.4) (layer "B.Cu") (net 1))
 (segment (start 61.5 71) (end 61.5 70.6) (width 0.4) (layer "B.Cu") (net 1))
 (segment (start 61.5 70.6) (end 61.55 70.55) (width 0.4) (layer "B.Cu") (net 1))
 (segment (start 61.55 70.55) (end 61.55 70.5) (width 0.4) (layer "B.Cu") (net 1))
 (segment (start 61.55 70.5) (end 61.6 70.45) (width 0.4) (layer "B.Cu") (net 1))
 (segment (start 61.6 70.45) (end 61.6 70.4) (width 0.4) (layer "B.Cu") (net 1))
 (segment (start 61.6 70.4) (end 61.75 70.25) (width 0.4) (layer "B.Cu") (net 1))
 (segment (start 61.75 70.25) (end 61.8 70.25) (width 0.4) (layer "B.Cu") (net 1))
 (segment (start 61.8 70.25) (end 61.85 70.2) (width 0.4) (layer "B.Cu") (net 1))
 (segment (start 61.85 70.2) (end 61.9 70.2) (width 0.4) (layer "B.Cu") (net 1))
 (segment (start 61.9 70.2) (end 61.95 70.15) (width 0.4) (layer "B.Cu") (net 1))
 (segment (start 61.95 70.15) (end 64.35 70.15) (width 0.4) (layer "B.Cu") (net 1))
 (segment (start 64.35 70.15) (end 64.4 70.2) (width 0.4) (layer "B.Cu") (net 1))
 (segment (start 64.4 70.2) (end 64.45 70.2) (width 0.4) (layer "B.Cu") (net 1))
 (segment (start 64.45 70.2) (end 64.5 70.25) (width 0.4) (layer "B.Cu") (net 1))
 (segment (start 64.5 70.25) (end 64.55 70.25) (width 0.4) (layer "B.Cu") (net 1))
 (segment (start 64.55 70.25) (end 64.6 70.3) (width 0.4) (layer "B.Cu") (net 1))
 (segment (start 64.6 70.3) (end 64.65 70.3) (width 0.4) (layer "B.Cu") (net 1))
 (segment (start 64.65 70.3) (end 64.7 70.35) (width 0.4) (layer "B.Cu") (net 1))
 (segment (start 64.7 70.35) (end 64.8 70.35) (width 0.4) (layer "B.Cu") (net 1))
 (segment (start 64.8 70.35) (end 64.85 70.4) (width 0.4) (layer "B.Cu") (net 1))
 (segment (start 64.85 70.4) (end 64.9 70.4) (width 0.4) (layer "B.Cu") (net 1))
 (segment (start 64.9 70.4) (end 64.95 70.45) (width 0.4) (layer "B.Cu") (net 1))
 (segment (start 64.95 70.45) (end 65 70.45) (width 0.4) (layer "B.Cu") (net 1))
 (segment (start 65 70.45) (end 65.05 70.5) (width 0.4) (layer "B.Cu") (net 1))
 (segment (start 65.05 70.5) (end 65.1 70.5) (width 0.4) (layer "B.Cu") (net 1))
 (segment (start 65.1 70.5) (end 65.15 70.55) (width 0.4) (layer "B.Cu") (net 1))
 (segment (start 65.15 70.55) (end 65.2 70.55) (width 0.4) (layer "B.Cu") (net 1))
 (segment (start 65.2 70.55) (end 65.25 70.6) (width 0.4) (layer "B.Cu") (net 1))
 (segment (start 65.25 70.6) (end 65.35 70.6) (width 0.4) (layer "B.Cu") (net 1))
 (segment (start 65.35 70.6) (end 65.4 70.65) (width 0.4) (layer "B.Cu") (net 1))
 (segment (start 65.4 70.65) (end 65.45 70.65) (width 0.4) (layer "B.Cu") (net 1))
 (segment (start 65.45 70.65) (end 65.5 70.7) (width 0.4) (layer "B.Cu") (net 1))
 (segment (start 65.5 70.7) (end 67.25 70.7) (width 0.4) (layer "B.Cu") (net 1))
 (segment (start 67.25 70.7) (end 67.4 70.85) (width 0.4) (layer "F.Cu") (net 1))
 (segment (start 67.4 70.85) (end 67.4 70.9) (width 0.4) (layer "F.Cu") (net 1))
 (segment (start 67.4 70.9) (end 67.5 71) (width 0.4) (layer "F.Cu") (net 1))
 (segment (start 67.5 71) (end 67.5 71.3) (width 0.4) (layer "F.Cu") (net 1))
 (segment (start 67.5 71.3) (end 67.6 71.645) (width 0.4) (layer "F.Cu") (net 1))
 (via (at 67.25 70.7) (size 0.5) (drill 0.3) (layers "F.Cu" "B.Cu") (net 1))
 (segment (start 67.415 73.3) (end 67.45 73.15) (width 0.25) (layer "F.Cu") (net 1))
 (segment (start 67.45 73.15) (end 67.45 72) (width 0.25) (layer "F.Cu") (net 1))
 (segment (start 67.45 72) (end 67.6 71.645) (width 0.25) (layer "F.Cu") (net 1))
 (segment (start 61.385 73.3) (end 61.35 73.15) (width 0.25) (layer "F.Cu") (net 1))
 (segment (start 61.35 73.15) (end 61.35 72) (width 0.25) (layer "F.Cu") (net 1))
 (segment (start 61.35 72) (end 61.2 71.645) (width 0.25) (layer "F.Cu") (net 1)))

